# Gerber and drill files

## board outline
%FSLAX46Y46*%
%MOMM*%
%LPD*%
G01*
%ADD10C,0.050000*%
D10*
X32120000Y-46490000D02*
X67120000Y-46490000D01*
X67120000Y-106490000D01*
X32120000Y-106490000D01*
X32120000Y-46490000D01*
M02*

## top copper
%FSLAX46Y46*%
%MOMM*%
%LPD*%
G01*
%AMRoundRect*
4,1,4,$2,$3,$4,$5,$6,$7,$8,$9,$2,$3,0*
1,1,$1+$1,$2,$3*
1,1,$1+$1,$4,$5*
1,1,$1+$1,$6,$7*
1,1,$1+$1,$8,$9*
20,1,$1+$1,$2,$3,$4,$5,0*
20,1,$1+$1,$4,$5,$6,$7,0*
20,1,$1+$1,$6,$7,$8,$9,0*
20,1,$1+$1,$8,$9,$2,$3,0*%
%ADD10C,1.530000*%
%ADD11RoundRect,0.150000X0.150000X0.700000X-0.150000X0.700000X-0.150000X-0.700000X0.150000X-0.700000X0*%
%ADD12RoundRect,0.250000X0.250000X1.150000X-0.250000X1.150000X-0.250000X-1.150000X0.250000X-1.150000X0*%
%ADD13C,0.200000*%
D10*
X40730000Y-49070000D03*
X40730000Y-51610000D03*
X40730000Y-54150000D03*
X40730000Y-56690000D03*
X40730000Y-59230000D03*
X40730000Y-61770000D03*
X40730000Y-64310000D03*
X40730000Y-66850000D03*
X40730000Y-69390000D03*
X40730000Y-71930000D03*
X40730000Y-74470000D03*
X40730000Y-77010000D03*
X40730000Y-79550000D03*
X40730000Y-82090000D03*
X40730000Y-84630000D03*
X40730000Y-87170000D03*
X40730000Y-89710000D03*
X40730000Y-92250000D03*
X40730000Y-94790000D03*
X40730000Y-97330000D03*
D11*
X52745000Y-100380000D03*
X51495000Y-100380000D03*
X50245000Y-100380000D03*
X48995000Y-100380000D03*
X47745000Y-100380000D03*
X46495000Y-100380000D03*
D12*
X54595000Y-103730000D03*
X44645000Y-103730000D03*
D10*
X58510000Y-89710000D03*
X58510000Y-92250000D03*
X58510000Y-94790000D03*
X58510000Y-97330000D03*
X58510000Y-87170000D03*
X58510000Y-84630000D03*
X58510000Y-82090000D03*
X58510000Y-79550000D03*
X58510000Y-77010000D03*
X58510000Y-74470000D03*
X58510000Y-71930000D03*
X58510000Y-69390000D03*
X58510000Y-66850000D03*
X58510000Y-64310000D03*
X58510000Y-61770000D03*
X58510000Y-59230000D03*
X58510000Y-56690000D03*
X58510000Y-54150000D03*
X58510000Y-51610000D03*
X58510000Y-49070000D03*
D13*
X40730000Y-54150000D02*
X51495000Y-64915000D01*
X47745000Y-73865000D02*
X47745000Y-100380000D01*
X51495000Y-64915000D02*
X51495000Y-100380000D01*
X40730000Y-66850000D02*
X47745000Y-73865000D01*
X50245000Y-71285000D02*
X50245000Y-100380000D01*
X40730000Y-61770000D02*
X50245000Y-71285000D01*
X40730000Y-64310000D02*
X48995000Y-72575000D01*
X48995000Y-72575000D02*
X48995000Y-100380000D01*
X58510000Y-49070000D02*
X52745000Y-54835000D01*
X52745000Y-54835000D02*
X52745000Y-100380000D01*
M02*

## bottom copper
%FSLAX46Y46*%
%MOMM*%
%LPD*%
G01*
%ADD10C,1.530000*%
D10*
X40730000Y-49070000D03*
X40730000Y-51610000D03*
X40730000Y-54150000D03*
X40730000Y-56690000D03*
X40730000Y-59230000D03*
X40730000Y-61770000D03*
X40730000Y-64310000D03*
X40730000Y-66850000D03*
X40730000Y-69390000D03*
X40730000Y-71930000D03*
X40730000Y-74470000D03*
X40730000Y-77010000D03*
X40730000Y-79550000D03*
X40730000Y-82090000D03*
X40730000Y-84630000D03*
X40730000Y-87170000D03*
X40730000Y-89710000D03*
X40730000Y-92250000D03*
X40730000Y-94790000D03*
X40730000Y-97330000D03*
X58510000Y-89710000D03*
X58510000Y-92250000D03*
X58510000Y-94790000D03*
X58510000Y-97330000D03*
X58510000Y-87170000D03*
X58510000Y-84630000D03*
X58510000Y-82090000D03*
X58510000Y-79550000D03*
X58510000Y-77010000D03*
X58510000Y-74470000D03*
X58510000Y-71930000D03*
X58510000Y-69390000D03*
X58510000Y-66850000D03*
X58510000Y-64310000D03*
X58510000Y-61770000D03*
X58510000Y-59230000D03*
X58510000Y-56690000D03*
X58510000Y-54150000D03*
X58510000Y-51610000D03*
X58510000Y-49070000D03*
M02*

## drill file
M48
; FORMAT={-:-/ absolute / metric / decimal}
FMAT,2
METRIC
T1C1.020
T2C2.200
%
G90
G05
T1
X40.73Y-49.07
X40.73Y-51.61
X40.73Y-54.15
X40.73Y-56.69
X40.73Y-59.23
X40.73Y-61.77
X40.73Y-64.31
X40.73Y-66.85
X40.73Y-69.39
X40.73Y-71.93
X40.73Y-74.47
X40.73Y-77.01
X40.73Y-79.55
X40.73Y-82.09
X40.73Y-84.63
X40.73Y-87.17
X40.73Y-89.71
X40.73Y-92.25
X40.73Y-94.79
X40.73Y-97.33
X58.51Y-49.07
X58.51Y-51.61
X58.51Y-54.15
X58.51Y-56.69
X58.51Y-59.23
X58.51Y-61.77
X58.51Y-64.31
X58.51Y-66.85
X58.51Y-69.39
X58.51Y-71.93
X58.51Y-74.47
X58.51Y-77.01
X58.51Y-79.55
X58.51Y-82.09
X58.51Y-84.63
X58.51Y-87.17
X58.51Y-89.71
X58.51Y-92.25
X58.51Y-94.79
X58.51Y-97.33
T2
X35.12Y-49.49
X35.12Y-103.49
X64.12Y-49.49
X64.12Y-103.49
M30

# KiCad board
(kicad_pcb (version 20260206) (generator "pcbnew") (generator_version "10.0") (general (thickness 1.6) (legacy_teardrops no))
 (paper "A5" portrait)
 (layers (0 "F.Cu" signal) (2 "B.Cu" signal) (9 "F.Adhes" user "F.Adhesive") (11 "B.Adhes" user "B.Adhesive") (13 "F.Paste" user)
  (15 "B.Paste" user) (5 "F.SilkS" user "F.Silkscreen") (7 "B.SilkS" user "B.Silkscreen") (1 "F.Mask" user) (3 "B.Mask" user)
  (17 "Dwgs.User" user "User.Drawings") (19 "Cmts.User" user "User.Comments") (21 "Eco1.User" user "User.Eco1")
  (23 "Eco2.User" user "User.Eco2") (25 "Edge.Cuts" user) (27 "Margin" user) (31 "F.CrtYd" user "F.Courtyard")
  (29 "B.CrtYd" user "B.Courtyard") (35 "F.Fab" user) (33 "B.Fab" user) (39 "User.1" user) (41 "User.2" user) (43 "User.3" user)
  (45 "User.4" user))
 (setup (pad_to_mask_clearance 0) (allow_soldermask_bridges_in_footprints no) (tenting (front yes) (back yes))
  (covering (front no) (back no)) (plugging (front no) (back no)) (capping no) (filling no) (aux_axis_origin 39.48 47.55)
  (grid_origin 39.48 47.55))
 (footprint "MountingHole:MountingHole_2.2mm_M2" (layer "F.Cu") (at 35.12 49.49)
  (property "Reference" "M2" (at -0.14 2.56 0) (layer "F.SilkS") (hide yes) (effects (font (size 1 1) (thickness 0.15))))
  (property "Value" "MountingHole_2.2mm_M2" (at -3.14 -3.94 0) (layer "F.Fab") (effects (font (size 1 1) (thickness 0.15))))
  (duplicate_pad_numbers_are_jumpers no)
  (pad "" np_thru_hole circle (at 0 0) (size 2.2 2.2) (drill 2.2) (layers "*.Cu" "*.Mask")))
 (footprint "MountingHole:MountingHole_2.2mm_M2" (layer "F.Cu") (at 64.12 49.49)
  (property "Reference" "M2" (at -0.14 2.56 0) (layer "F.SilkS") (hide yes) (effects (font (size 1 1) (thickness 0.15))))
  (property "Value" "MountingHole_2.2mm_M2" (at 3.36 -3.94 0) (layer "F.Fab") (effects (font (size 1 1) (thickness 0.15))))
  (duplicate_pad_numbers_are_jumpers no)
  (pad "" np_thru_hole circle (at 0 0) (size 2.2 2.2) (drill 2.2) (layers "*.Cu" "*.Mask")))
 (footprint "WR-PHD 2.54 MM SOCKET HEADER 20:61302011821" (layer "F.Cu") (at 40.73 73.2 -90)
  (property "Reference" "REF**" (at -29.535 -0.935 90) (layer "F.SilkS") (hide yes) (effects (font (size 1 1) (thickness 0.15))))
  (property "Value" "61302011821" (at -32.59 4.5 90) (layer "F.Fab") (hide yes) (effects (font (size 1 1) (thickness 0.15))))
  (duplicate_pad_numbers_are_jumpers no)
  (pad "1" thru_hole circle (at -24.13 0 270) (size 1.53 1.53) (drill 1.02) (layers "*.Cu" "*.Mask") (remove_unused_layers no)
   (solder_mask_margin 0.102))
  (pad "2" thru_hole circle (at -21.59 0 270) (size 1.53 1.53) (drill 1.02) (layers "*.Cu" "*.Mask") (remove_unused_layers no)
   (solder_mask_margin 0.102))
  (pad "3" thru_hole circle (at -19.05 0 270) (size 1.53 1.53) (drill 1.02) (layers "*.Cu" "*.Mask") (remove_unused_layers no) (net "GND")
   (solder_mask_margin 0.102))
  (pad "4" thru_hole circle (at -16.51 0 270) (size 1.53 1.53) (drill 1.02) (layers "*.Cu" "*.Mask") (remove_unused_layers no)
   (solder_mask_margin 0.102))
  (pad "5" thru_hole circle (at -13.97 0 270) (size 1.53 1.53) (drill 1.02) (layers "*.Cu" "*.Mask") (remove_unused_layers no)
   (solder_mask_margin 0.102))
  (pad "6" thru_hole circle (at -11.43 0 270) (size 1.53 1.53) (drill 1.02) (layers "*.Cu" "*.Mask") (remove_unused_layers no) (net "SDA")
   (solder_mask_margin 0.102))
  (pad "7" thru_hole circle (at -8.89 0 270) (size 1.53 1.53) (drill 1.02) (layers "*.Cu" "*.Mask") (remove_unused_layers no) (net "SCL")
   (solder_mask_margin 0.102))
  (pad "8" thru_hole circle (at -6.35 0 270) (size 1.53 1.53) (drill 1.02) (layers "*.Cu" "*.Mask") (remove_unused_layers no) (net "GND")
   (solder_mask_margin 0.102))
  (pad "9" thru_hole circle (at -3.81 0 270) (size 1.53 1.53) (drill 1.02) (layers "*.Cu" "*.Mask") (remove_unused_layers no)
   (solder_mask_margin 0.102))
  (pad "10" thru_hole circle (at -1.27 0 270) (size 1.53 1.53) (drill 1.02) (layers "*.Cu" "*.Mask") (remove_unused_layers no)
   (solder_mask_margin 0.102))
  (pad "11" thru_hole circle (at 1.27 0 270) (size 1.53 1.53) (drill 1.02) (layers "*.Cu" "*.Mask") (remove_unused_layers no)
   (solder_mask_margin 0.102))
  (pad "12" thru_hole circle (at 3.81 0 270) (size 1.53 1.53) (drill 1.02) (layers "*.Cu" "*.Mask") (remove_unused_layers no)
   (solder_mask_margin 0.102))
  (pad "13" thru_hole circle (at 6.35 0 270) (size 1.53 1.53) (drill 1.02) (layers "*.Cu" "*.Mask") (remove_unused_layers no)
   (solder_mask_margin 0.102))
  (pad "14" thru_hole circle (at 8.89 0 270) (size 1.53 1.53) (drill 1.02) (layers "*.Cu" "*.Mask") (remove_unused_layers no)
   (solder_mask_margin 0.102))
  (pad "15" thru_hole circle (at 11.43 0 270) (size 1.53 1.53) (drill 1.02) (layers "*.Cu" "*.Mask") (remove_unused_layers no)
   (solder_mask_margin 0.102))
  (pad "16" thru_hole circle (at 13.97 0 270) (size 1.53 1.53) (drill 1.02) (layers "*.Cu" "*.Mask") (remove_unused_layers no)
   (solder_mask_margin 0.102))
  (pad "17" thru_hole circle (at 16.51 0 270) (size 1.53 1.53) (drill 1.02) (layers "*.Cu" "*.Mask") (remove_unused_layers no)
   (solder_mask_margin 0.102))
  (pad "18" thru_hole circle (at 19.05 0 270) (size 1.53 1.53) (drill 1.02) (layers "*.Cu" "*.Mask") (remove_unused_layers no)
   (solder_mask_margin 0.102))
  (pad "19" thru_hole circle (at 21.59 0 270) (size 1.53 1.53) (drill 1.02) (layers "*.Cu" "*.Mask") (remove_unused_layers no)
   (solder_mask_margin 0.102))
  (pad "20" thru_hole circle (at 24.13 0 270) (size 1.53 1.53) (drill 1.02) (layers "*.Cu" "*.Mask") (remove_unused_layers no)
   (solder_mask_margin 0.102)))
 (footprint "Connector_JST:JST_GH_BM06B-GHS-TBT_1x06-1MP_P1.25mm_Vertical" (layer "F.Cu") (at 49.62 102.33 180)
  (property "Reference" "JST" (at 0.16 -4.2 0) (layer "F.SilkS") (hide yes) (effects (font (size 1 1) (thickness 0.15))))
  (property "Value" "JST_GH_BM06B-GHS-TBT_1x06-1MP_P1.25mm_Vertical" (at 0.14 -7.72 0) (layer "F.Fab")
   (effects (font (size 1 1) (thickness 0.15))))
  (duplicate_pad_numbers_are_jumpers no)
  (pad "1" smd roundrect (at -3.125 1.95 180) (size 0.6 1.7) (layers "F.Cu" "F.Mask" "F.Paste") (roundrect_rratio 0.25) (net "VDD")
   (solder_mask_margin 0))
  (pad "2" smd roundrect (at -1.875 1.95 180) (size 0.6 1.7) (layers "F.Cu" "F.Mask" "F.Paste") (roundrect_rratio 0.25) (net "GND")
   (solder_mask_margin 0))
  (pad "3" smd roundrect (at -0.625 1.95 180) (size 0.6 1.7) (layers "F.Cu" "F.Mask" "F.Paste") (roundrect_rratio 0.25) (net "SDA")
   (solder_mask_margin 0))
  (pad "4" smd roundrect (at 0.625 1.95 180) (size 0.6 1.7) (layers "F.Cu" "F.Mask" "F.Paste") (roundrect_rratio 0.25) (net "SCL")
   (solder_mask_margin 0))
  (pad "5" smd roundrect (at 1.875 1.95 180) (size 0.6 1.7) (layers "F.Cu" "F.Mask" "F.Paste") (roundrect_rratio 0.25) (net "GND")
   (solder_mask_margin 0))
  (pad "6" smd roundrect (at 3.125 1.95 180) (size 0.6 1.7) (layers "F.Cu" "F.Mask" "F.Paste") (roundrect_rratio 0.25))
  (pad "MP" smd roundrect (at -4.975 -1.4 180) (size 1 2.8) (layers "F.Cu" "F.Mask" "F.Paste") (roundrect_rratio 0.25))
  (pad "MP" smd roundrect (at 4.975 -1.4 180) (size 1 2.8) (layers "F.Cu" "F.Mask" "F.Paste") (roundrect_rratio 0.25)))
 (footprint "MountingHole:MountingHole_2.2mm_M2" (layer "F.Cu") (at 35.12 103.49)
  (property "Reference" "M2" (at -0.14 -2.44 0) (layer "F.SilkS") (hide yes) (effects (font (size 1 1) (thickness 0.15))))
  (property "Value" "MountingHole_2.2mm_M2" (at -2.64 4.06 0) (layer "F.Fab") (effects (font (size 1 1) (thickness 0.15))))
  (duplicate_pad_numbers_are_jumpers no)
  (pad "" np_thru_hole circle (at 0 0) (size 2.2 2.2) (drill 2.2) (layers "*.Cu" "*.Mask")))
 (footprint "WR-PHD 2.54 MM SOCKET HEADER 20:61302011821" (layer "F.Cu") (at 58.51 73.2 -90)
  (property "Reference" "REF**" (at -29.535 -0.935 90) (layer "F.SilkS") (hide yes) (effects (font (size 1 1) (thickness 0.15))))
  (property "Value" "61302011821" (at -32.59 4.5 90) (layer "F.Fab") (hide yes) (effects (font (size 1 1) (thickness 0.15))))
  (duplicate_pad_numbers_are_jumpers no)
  (pad "17" thru_hole circle (at 16.51 0 270) (size 1.53 1.53) (drill 1.02) (layers "*.Cu" "*.Mask") (remove_unused_layers no)
   (solder_mask_margin 0.102))
  (pad "18" thru_hole circle (at 19.05 0 270) (size 1.53 1.53) (drill 1.02) (layers "*.Cu" "*.Mask") (remove_unused_layers no)
   (solder_mask_margin 0.102))
  (pad "19" thru_hole circle (at 21.59 0 270) (size 1.53 1.53) (drill 1.02) (layers "*.Cu" "*.Mask") (remove_unused_layers no)
   (solder_mask_margin 0.102))
  (pad "20" thru_hole circle (at 24.13 0 270) (size 1.53 1.53) (drill 1.02) (layers "*.Cu" "*.Mask") (remove_unused_layers no)
   (solder_mask_margin 0.102))
  (pad "25" thru_hole circle (at 13.97 0 270) (size 1.53 1.53) (drill 1.02) (layers "*.Cu" "*.Mask") (remove_unused_layers no)
   (solder_mask_margin 0.102))
  (pad "26" thru_hole circle (at 11.43 0 270) (size 1.53 1.53) (drill 1.02) (layers "*.Cu" "*.Mask") (remove_unused_layers no)
   (solder_mask_margin 0.102))
  (pad "27" thru_hole circle (at 8.89 0 270) (size 1.53 1.53) (drill 1.02) (layers "*.Cu" "*.Mask") (remove_unused_layers no)
   (solder_mask_margin 0.102))
  (pad "28" thru_hole circle (at 6.35 0 270) (size 1.53 1.53) (drill 1.02) (layers "*.Cu" "*.Mask") (remove_unused_layers no)
   (solder_mask_margin 0.102))
  (pad "29" thru_hole circle (at 3.81 0 270) (size 1.53 1.53) (drill 1.02) (layers "*.Cu" "*.Mask") (remove_unused_layers no)
   (solder_mask_margin 0.102))
  (pad "30" thru_hole circle (at 1.27 0 270) (size 1.53 1.53) (drill 1.02) (layers "*.Cu" "*.Mask") (remove_unused_layers no)
   (solder_mask_margin 0.102))
  (pad "31" thru_hole circle (at -1.27 0 270) (size 1.53 1.53) (drill 1.02) (layers "*.Cu" "*.Mask") (remove_unused_layers no)
   (solder_mask_margin 0.102))
  (pad "32" thru_hole circle (at -3.81 0 270) (size 1.53 1.53) (drill 1.02) (layers "*.Cu" "*.Mask") (remove_unused_layers no)
   (solder_mask_margin 0.102))
  (pad "33" thru_hole circle (at -6.35 0 270) (size 1.53 1.53) (drill 1.02) (layers "*.Cu" "*.Mask") (remove_unused_layers no)
   (solder_mask_margin 0.102))
  (pad "34" thru_hole circle (at -8.89 0 270) (size 1.53 1.53) (drill 1.02) (layers "*.Cu" "*.Mask") (remove_unused_layers no)
   (solder_mask_margin 0.102))
  (pad "35" thru_hole circle (at -11.43 0 270) (size 1.53 1.53) (drill 1.02) (layers "*.Cu" "*.Mask") (remove_unused_layers no)
   (solder_mask_margin 0.102))
  (pad "36" thru_hole circle (at -13.97 0 270) (size 1.53 1.53) (drill 1.02) (layers "*.Cu" "*.Mask") (remove_unused_layers no)
   (solder_mask_margin 0.102))
  (pad "37" thru_hole circle (at -16.51 0 270) (size 1.53 1.53) (drill 1.02) (layers "*.Cu" "*.Mask") (remove_unused_layers no)
   (solder_mask_margin 0.102))
  (pad "38" thru_hole circle (at -19.05 0 270) (size 1.53 1.53) (drill 1.02) (layers "*.Cu" "*.Mask") (remove_unused_layers no)
   (solder_mask_margin 0.102))
  (pad "39" thru_hole circle (at -21.59 0 270) (size 1.53 1.53) (drill 1.02) (layers "*.Cu" "*.Mask") (remove_unused_layers no)
   (solder_mask_margin 0.102))
  (pad "40" thru_hole circle (at -24.13 0 270) (size 1.53 1.53) (drill 1.02) (layers "*.Cu" "*.Mask") (remove_unused_layers no) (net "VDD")
   (solder_mask_margin 0.102)))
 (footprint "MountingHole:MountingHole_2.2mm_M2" (layer "F.Cu") (at 64.12 103.49)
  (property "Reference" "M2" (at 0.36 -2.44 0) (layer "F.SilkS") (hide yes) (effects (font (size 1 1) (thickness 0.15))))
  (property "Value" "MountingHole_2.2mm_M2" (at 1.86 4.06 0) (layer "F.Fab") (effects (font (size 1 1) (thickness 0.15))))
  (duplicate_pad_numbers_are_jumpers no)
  (pad "" np_thru_hole circle (at 0 0) (size 2.2 2.2) (drill 2.2) (layers "*.Cu" "*.Mask")))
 (gr_rect (start 32.12 46.49) (end 67.12 106.49) (stroke (width 0.05) (type solid)) (fill no) (layer "Edge.Cuts"))
 (segment (start 40.73 54.15) (end 51.495 64.915) (width 0.2) (layer "F.Cu") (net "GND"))
 (segment (start 47.745 73.865) (end 47.745 100.38) (width 0.2) (layer "F.Cu") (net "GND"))
 (segment (start 51.495 64.915) (end 51.495 100.38) (width 0.2) (layer "F.Cu") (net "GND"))
 (segment (start 40.73 66.85) (end 47.745 73.865) (width 0.2) (layer "F.Cu") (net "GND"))
 (segment (start 50.245 71.285) (end 50.245 100.38) (width 0.2) (layer "F.Cu") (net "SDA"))
 (segment (start 40.73 61.77) (end 50.245 71.285) (width 0.2) (layer "F.Cu") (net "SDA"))
 (segment (start 40.73 64.31) (end 48.995 72.575) (width 0.2) (layer "F.Cu") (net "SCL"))
 (segment (start 48.995 72.575) (end 48.995 100.38) (width 0.2) (layer "F.Cu") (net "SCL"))
 (segment (start 58.51 49.07) (end 52.745 54.835) (width 0.2) (layer "F.Cu") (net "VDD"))
 (segment (start 52.745 54.835) (end 52.745 100.38) (width 0.2) (layer "F.Cu") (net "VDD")))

